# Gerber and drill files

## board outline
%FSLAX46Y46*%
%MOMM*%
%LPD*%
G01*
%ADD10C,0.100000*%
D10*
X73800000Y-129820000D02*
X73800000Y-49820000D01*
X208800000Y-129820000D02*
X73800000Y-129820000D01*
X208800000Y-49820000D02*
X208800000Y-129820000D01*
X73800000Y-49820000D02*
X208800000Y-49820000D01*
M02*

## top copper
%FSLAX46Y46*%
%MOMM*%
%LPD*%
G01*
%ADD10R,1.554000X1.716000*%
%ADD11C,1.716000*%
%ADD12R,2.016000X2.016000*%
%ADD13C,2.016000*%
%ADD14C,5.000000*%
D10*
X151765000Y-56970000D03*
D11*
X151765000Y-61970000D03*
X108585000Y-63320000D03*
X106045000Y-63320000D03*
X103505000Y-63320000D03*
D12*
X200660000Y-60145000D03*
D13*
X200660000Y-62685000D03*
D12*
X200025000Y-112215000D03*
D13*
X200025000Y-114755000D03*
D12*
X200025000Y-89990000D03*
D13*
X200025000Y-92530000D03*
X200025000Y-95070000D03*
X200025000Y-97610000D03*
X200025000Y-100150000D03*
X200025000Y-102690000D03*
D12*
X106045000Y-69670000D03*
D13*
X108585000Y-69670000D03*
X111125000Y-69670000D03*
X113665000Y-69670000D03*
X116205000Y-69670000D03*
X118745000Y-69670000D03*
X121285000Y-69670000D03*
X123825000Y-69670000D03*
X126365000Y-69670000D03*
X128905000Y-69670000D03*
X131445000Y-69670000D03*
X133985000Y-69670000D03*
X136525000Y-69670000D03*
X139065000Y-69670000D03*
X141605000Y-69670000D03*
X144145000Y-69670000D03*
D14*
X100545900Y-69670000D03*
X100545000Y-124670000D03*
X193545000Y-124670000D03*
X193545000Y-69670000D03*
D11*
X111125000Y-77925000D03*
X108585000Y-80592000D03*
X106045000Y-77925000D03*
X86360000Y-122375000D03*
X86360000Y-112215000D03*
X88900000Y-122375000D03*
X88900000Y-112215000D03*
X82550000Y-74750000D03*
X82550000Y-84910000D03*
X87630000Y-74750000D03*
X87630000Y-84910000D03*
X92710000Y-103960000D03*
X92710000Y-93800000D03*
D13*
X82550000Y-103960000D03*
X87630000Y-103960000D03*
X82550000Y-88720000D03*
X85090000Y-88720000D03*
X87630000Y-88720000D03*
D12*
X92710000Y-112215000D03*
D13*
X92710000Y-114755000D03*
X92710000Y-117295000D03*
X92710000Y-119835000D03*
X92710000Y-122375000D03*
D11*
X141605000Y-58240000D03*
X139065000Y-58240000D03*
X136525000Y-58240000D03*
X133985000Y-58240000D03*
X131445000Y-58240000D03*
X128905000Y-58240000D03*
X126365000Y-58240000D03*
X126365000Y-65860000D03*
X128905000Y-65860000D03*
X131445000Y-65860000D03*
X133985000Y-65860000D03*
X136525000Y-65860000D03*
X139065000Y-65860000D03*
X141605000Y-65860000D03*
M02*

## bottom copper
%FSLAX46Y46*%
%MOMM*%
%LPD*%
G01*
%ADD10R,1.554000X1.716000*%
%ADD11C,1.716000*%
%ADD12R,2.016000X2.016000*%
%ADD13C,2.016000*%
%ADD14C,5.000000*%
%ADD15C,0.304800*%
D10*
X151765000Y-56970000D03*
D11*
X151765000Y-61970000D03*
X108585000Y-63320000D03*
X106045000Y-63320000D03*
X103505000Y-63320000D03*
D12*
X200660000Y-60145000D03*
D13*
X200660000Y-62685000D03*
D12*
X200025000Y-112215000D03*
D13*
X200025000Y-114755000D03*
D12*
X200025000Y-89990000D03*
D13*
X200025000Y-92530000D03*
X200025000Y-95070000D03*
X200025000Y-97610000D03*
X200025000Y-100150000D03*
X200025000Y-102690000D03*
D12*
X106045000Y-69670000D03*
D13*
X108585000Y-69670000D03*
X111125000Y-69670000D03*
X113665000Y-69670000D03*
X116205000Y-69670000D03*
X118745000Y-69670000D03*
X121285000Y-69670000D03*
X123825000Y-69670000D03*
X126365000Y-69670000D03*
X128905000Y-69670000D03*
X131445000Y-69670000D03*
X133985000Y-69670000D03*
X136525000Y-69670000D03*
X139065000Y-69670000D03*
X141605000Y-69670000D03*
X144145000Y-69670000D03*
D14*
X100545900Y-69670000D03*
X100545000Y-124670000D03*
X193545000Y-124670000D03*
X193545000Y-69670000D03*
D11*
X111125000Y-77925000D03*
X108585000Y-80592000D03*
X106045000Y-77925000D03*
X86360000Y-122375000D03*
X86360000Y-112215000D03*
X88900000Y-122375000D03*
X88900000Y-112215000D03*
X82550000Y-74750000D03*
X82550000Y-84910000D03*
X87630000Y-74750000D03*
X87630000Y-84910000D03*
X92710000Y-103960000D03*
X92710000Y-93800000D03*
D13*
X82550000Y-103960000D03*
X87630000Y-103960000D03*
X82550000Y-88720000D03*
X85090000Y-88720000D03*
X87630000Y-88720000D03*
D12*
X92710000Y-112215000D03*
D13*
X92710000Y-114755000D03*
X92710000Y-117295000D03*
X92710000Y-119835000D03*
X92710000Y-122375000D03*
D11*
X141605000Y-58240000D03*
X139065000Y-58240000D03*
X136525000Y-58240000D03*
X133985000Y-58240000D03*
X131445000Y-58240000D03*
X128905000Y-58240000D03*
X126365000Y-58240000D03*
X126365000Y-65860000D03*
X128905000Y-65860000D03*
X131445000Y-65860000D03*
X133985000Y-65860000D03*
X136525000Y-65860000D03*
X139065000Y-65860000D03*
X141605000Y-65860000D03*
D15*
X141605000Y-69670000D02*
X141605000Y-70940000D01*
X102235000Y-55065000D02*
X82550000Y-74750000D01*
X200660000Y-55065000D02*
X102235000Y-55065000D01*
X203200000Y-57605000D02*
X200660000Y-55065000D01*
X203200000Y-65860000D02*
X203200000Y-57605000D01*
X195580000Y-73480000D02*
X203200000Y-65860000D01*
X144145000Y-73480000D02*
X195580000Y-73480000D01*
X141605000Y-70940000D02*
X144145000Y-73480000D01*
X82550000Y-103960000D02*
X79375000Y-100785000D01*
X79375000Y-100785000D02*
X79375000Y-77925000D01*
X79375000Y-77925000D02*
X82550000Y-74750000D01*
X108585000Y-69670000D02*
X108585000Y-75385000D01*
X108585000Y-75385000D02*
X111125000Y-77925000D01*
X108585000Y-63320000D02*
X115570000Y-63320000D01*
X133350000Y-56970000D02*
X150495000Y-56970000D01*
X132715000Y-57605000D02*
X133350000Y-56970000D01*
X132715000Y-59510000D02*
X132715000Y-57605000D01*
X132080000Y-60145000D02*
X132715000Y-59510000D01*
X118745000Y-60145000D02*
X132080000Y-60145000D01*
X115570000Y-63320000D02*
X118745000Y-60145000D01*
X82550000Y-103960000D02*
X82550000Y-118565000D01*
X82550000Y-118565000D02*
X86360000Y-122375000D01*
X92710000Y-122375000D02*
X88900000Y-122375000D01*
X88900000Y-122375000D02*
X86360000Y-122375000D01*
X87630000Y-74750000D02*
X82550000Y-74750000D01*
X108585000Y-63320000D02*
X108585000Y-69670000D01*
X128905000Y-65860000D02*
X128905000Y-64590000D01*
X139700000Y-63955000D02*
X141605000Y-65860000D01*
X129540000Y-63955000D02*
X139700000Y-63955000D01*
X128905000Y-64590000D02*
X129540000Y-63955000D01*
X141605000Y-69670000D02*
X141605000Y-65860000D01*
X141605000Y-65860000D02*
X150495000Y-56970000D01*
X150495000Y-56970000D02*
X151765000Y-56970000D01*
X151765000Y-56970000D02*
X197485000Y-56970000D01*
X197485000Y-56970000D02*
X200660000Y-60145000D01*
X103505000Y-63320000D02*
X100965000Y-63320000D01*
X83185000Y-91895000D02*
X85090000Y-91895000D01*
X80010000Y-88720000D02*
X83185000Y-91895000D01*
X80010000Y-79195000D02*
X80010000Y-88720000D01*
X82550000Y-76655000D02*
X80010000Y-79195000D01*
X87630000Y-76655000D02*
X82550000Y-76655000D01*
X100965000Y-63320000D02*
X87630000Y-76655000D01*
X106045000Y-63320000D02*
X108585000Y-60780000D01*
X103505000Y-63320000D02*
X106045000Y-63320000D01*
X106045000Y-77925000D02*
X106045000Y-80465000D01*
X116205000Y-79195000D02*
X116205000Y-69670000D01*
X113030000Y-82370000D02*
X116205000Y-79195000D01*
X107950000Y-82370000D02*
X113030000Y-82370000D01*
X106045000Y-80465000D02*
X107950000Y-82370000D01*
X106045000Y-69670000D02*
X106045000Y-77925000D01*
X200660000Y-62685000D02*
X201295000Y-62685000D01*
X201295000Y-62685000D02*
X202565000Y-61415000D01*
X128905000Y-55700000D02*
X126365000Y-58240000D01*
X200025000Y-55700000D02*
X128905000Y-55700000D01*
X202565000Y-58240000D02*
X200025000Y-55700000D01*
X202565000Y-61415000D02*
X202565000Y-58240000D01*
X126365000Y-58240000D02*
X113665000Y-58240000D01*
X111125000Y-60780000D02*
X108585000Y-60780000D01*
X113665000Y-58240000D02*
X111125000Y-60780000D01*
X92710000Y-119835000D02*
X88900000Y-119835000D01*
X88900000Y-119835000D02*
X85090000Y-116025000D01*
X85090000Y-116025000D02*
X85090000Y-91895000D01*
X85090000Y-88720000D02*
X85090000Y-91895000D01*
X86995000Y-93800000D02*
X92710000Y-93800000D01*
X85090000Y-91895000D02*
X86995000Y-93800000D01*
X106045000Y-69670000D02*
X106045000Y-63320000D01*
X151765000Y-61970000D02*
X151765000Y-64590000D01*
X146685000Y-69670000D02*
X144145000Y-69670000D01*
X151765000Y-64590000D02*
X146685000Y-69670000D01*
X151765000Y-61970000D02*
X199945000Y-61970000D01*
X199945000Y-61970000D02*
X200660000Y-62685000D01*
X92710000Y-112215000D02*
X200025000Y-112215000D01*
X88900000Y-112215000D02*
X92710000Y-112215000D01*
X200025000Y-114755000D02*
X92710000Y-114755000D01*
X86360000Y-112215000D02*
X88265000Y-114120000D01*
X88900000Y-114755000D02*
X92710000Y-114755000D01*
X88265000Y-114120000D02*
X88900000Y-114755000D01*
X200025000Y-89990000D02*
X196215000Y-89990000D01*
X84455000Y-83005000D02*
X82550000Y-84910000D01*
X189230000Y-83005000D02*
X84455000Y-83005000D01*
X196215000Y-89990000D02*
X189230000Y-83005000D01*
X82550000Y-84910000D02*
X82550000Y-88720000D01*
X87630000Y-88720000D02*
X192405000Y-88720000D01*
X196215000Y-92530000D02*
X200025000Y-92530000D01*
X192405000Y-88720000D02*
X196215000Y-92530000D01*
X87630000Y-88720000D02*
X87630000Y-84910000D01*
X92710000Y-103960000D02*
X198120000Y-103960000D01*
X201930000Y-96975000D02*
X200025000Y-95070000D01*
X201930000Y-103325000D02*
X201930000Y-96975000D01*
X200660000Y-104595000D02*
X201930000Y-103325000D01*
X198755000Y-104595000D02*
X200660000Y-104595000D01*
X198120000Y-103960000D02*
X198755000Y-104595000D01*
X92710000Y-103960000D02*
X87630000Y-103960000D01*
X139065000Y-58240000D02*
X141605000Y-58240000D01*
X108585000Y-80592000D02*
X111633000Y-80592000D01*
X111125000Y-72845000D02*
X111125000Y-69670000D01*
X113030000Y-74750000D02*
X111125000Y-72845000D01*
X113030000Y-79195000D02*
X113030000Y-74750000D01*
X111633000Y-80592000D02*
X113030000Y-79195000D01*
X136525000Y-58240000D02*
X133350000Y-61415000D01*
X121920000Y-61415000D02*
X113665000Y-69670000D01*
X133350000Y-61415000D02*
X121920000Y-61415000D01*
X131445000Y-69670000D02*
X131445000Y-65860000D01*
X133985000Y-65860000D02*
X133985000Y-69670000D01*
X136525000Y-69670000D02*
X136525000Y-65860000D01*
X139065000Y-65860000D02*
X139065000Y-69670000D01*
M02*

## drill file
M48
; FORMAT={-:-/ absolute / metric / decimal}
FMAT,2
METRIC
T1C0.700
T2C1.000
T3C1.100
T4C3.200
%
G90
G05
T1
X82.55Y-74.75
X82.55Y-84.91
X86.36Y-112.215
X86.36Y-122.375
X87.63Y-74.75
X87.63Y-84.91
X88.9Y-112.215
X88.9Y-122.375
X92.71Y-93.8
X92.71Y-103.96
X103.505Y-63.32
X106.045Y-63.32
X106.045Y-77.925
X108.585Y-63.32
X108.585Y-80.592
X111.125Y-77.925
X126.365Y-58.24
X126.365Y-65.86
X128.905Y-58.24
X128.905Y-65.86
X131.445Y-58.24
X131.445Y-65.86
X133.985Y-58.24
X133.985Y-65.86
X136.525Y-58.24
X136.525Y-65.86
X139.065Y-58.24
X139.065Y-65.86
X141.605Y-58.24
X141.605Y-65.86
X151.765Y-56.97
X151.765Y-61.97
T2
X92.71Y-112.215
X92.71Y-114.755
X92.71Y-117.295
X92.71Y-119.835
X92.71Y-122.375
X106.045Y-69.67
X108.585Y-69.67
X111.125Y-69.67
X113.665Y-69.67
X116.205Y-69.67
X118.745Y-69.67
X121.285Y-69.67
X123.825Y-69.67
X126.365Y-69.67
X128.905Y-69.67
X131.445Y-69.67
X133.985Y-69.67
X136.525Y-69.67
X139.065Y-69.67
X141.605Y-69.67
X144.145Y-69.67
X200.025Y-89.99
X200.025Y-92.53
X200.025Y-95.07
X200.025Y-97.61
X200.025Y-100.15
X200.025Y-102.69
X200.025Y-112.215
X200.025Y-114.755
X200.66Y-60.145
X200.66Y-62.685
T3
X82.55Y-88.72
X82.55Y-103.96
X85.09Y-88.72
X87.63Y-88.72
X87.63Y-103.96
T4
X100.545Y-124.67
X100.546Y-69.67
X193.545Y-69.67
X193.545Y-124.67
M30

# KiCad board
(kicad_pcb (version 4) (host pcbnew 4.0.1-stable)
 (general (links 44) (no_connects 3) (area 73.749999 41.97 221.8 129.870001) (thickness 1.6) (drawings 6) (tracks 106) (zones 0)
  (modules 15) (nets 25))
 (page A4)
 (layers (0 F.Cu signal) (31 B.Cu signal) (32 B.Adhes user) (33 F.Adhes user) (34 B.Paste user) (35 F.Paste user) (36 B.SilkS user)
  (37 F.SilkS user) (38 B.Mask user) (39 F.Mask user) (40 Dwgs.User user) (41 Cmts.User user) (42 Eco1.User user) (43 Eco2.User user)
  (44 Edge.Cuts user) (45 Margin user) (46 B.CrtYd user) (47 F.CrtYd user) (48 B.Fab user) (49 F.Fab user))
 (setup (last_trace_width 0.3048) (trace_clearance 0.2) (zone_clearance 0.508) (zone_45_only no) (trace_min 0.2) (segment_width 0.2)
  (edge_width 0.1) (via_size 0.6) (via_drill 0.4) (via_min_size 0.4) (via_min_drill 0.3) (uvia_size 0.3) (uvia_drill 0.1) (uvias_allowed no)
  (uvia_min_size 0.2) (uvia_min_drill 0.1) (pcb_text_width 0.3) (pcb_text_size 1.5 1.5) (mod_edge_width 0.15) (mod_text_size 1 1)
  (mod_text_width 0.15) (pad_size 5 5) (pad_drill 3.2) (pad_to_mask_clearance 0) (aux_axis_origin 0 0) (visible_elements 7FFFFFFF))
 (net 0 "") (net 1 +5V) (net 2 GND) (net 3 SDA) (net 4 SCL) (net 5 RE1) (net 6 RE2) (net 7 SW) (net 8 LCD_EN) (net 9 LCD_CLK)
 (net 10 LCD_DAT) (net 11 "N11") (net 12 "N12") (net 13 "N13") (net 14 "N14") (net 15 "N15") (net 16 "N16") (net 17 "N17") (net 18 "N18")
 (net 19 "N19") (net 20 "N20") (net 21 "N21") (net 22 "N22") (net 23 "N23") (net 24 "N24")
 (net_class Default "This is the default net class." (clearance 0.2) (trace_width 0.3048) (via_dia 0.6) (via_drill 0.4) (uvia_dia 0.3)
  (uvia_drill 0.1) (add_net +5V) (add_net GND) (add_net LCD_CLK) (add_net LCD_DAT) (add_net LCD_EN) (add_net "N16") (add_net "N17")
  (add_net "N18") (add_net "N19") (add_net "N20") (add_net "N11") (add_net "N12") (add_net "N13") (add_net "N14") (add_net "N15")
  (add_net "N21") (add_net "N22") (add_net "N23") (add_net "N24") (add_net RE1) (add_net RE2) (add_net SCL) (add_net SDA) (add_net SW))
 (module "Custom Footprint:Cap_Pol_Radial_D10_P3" (layer F.Cu) (at 151.765 56.97 270)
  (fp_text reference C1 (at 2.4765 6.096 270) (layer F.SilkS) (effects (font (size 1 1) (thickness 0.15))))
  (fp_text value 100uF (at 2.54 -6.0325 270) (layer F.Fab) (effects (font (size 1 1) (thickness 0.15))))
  (pad 1 thru_hole rect (at 0 0 270) (size 1.716 1.554) (drill 0.7) (layers *.Cu *.Mask F.SilkS) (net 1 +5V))
  (pad 2 thru_hole circle (at 5 0 270) (size 1.716 1.716) (drill 0.7) (layers *.Cu *.Mask F.SilkS) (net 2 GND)))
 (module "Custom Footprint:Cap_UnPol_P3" (layer F.Cu) (at 108.585 63.32 270)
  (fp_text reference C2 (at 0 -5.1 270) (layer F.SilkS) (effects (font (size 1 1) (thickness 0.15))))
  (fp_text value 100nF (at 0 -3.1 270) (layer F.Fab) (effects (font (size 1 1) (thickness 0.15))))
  (pad 1 thru_hole circle (at 0 0 270) (size 1.716 1.716) (drill 0.7) (layers *.Cu *.Mask F.SilkS) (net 1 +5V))
  (pad 2 thru_hole circle (at 0 2.54 270) (size 1.716 1.716) (drill 0.7) (layers *.Cu *.Mask F.SilkS) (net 2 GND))
  (pad 2 thru_hole circle (at 0 5.08 270) (size 1.716 1.716) (drill 0.7) (layers *.Cu *.Mask F.SilkS) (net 2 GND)))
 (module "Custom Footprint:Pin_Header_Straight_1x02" (layer F.Cu) (at 200.66 60.145)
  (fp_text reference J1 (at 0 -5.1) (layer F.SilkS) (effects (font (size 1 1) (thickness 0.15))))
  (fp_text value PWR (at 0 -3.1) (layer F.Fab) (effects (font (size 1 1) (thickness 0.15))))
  (pad 1 thru_hole rect (at 0 0) (size 2.016 2.016) (drill 1) (layers *.Cu *.Mask F.SilkS) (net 1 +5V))
  (pad 2 thru_hole circle (at 0 2.54) (size 2.016 2.016) (drill 1) (layers *.Cu *.Mask F.SilkS) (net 2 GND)))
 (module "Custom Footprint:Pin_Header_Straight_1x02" (layer F.Cu) (at 200.025 112.215)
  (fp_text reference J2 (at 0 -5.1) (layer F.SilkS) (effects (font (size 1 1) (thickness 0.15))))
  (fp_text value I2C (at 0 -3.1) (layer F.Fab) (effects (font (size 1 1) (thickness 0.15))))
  (pad 1 thru_hole rect (at 0 0) (size 2.016 2.016) (drill 1) (layers *.Cu *.Mask F.SilkS) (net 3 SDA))
  (pad 2 thru_hole circle (at 0 2.54) (size 2.016 2.016) (drill 1) (layers *.Cu *.Mask F.SilkS) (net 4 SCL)))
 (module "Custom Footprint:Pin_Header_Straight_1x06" (layer F.Cu) (at 200.025 89.99)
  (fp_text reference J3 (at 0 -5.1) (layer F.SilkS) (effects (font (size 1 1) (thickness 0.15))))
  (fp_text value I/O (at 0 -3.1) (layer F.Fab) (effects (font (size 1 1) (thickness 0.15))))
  (pad 1 thru_hole rect (at 0 0) (size 2.016 2.016) (drill 1) (layers *.Cu *.Mask F.SilkS) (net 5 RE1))
  (pad 2 thru_hole circle (at 0 2.54) (size 2.016 2.016) (drill 1) (layers *.Cu *.Mask F.SilkS) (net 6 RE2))
  (pad 3 thru_hole circle (at 0 5.08) (size 2.016 2.016) (drill 1) (layers *.Cu *.Mask F.SilkS) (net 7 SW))
  (pad 4 thru_hole circle (at 0 7.62) (size 2.016 2.016) (drill 1) (layers *.Cu *.Mask F.SilkS) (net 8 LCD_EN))
  (pad 5 thru_hole circle (at 0 10.16) (size 2.016 2.016) (drill 1) (layers *.Cu *.Mask F.SilkS) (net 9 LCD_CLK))
  (pad 6 thru_hole circle (at 0 12.7) (size 2.016 2.016) (drill 1) (layers *.Cu *.Mask F.SilkS) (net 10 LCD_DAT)))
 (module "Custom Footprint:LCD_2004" (layer F.Cu) (at 106.045 69.67)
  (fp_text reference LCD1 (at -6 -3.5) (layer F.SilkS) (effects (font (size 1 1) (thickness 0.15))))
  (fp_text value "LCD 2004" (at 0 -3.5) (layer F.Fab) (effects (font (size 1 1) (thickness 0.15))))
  (pad 1 thru_hole rect (at 0 0) (size 2.016 2.016) (drill 1) (layers *.Cu *.Mask F.SilkS) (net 2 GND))
  (pad 2 thru_hole circle (at 2.54 0) (size 2.016 2.016) (drill 1) (layers *.Cu *.Mask F.SilkS) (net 1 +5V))
  (pad 3 thru_hole circle (at 5.08 0) (size 2.016 2.016) (drill 1) (layers *.Cu *.Mask F.SilkS) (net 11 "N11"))
  (pad 4 thru_hole circle (at 7.62 0) (size 2.016 2.016) (drill 1) (layers *.Cu *.Mask F.SilkS) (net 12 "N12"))
  (pad 5 thru_hole circle (at 10.16 0) (size 2.016 2.016) (drill 1) (layers *.Cu *.Mask F.SilkS) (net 2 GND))
  (pad 6 thru_hole circle (at 12.7 0) (size 2.016 2.016) (drill 1) (layers *.Cu *.Mask F.SilkS) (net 8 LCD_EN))
  (pad 7 thru_hole circle (at 15.24 0) (size 2.016 2.016) (drill 1) (layers *.Cu *.Mask F.SilkS) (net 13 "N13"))
  (pad 8 thru_hole circle (at 17.78 0) (size 2.016 2.016) (drill 1) (layers *.Cu *.Mask F.SilkS) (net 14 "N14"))
  (pad 9 thru_hole circle (at 20.32 0) (size 2.016 2.016) (drill 1) (layers *.Cu *.Mask F.SilkS) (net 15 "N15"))
  (pad 10 thru_hole circle (at 22.86 0) (size 2.016 2.016) (drill 1) (layers *.Cu *.Mask F.SilkS) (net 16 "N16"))
  (pad 11 thru_hole circle (at 25.4 0) (size 2.016 2.016) (drill 1) (layers *.Cu *.Mask F.SilkS) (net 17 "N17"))
  (pad 12 thru_hole circle (at 27.94 0) (size 2.016 2.016) (drill 1) (layers *.Cu *.Mask F.SilkS) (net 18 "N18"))
  (pad 13 thru_hole circle (at 30.48 0) (size 2.016 2.016) (drill 1) (layers *.Cu *.Mask F.SilkS) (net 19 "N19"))
  (pad 14 thru_hole circle (at 33.02 0) (size 2.016 2.016) (drill 1) (layers *.Cu *.Mask F.SilkS) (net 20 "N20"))
  (pad 15 thru_hole circle (at 35.56 0) (size 2.016 2.016) (drill 1) (layers *.Cu *.Mask F.SilkS) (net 1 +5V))
  (pad 16 thru_hole circle (at 38.1 0) (size 2.016 2.016) (drill 1) (layers *.Cu *.Mask F.SilkS) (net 2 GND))
  (pad 0 thru_hole circle (at -5.4991 0) (size 5 5) (drill 3.2) (layers *.Cu *.Mask F.SilkS))
  (pad 0 thru_hole circle (at -5.5 55) (size 5 5) (drill 3.2) (layers *.Cu *.Mask F.SilkS))
  (pad 0 thru_hole circle (at 87.5 55) (size 5 5) (drill 3.2) (layers *.Cu *.Mask F.SilkS))
  (pad 0 thru_hole circle (at 87.5 0) (size 5 5) (drill 3.2) (layers *.Cu *.Mask F.SilkS)))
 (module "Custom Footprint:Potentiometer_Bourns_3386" (layer F.Cu) (at 111.125 77.925)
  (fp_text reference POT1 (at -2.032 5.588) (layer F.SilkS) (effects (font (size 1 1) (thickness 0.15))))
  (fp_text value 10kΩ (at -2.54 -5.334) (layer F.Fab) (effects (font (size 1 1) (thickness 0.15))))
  (pad 1 thru_hole circle (at 0 0) (size 1.716 1.716) (drill 0.7) (layers *.Cu *.Mask F.SilkS) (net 1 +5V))
  (pad 2 thru_hole circle (at -2.54 2.667) (size 1.716 1.716) (drill 0.7) (layers *.Cu *.Mask F.SilkS) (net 11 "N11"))
  (pad 3 thru_hole circle (at -5.08 0) (size 1.716 1.716) (drill 0.7) (layers *.Cu *.Mask F.SilkS) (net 2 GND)))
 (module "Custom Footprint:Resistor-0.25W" (layer F.Cu) (at 86.36 122.375 90)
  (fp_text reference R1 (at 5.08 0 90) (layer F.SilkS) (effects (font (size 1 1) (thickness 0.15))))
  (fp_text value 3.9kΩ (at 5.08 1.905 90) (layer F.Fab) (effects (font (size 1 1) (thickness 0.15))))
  (pad 1 thru_hole circle (at 0 0 90) (size 1.716 1.716) (drill 0.7) (layers *.Cu *.Mask F.SilkS) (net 1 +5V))
  (pad 2 thru_hole circle (at 10.16 0 90) (size 1.716 1.716) (drill 0.7) (layers *.Cu *.Mask F.SilkS) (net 4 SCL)))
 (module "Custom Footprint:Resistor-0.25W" (layer F.Cu) (at 88.9 122.375 90)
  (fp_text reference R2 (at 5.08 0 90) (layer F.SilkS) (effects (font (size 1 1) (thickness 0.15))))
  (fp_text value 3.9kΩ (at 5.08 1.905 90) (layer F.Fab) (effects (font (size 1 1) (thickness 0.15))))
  (pad 1 thru_hole circle (at 0 0 90) (size 1.716 1.716) (drill 0.7) (layers *.Cu *.Mask F.SilkS) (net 1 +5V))
  (pad 2 thru_hole circle (at 10.16 0 90) (size 1.716 1.716) (drill 0.7) (layers *.Cu *.Mask F.SilkS) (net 3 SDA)))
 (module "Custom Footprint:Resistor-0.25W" (layer F.Cu) (at 82.55 74.75 270)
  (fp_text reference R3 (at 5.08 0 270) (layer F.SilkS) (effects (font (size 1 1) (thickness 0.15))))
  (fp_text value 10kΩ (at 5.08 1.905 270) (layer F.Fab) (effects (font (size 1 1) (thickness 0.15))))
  (pad 1 thru_hole circle (at 0 0 270) (size 1.716 1.716) (drill 0.7) (layers *.Cu *.Mask F.SilkS) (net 1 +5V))
  (pad 2 thru_hole circle (at 10.16 0 270) (size 1.716 1.716) (drill 0.7) (layers *.Cu *.Mask F.SilkS) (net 5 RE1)))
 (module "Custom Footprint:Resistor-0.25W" (layer F.Cu) (at 87.63 74.75 270)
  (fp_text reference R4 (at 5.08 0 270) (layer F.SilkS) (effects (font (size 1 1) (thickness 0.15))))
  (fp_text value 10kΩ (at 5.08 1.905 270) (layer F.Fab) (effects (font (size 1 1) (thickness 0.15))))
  (pad 1 thru_hole circle (at 0 0 270) (size 1.716 1.716) (drill 0.7) (layers *.Cu *.Mask F.SilkS) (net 1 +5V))
  (pad 2 thru_hole circle (at 10.16 0 270) (size 1.716 1.716) (drill 0.7) (layers *.Cu *.Mask F.SilkS) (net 6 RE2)))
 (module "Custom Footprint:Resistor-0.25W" (layer F.Cu) (at 92.71 103.96 90)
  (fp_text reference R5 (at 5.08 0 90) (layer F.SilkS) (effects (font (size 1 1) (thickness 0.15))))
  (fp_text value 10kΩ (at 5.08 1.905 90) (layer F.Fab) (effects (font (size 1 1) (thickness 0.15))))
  (pad 1 thru_hole circle (at 0 0 90) (size 1.716 1.716) (drill 0.7) (layers *.Cu *.Mask F.SilkS) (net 7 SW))
  (pad 2 thru_hole circle (at 10.16 0 90) (size 1.716 1.716) (drill 0.7) (layers *.Cu *.Mask F.SilkS) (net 2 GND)))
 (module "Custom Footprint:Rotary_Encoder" (layer F.Cu) (at 85.09 98.88 180)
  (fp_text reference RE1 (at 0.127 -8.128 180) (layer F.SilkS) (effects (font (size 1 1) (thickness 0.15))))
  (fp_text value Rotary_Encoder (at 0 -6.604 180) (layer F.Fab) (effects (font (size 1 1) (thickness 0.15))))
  (pad 1 thru_hole circle (at 2.54 -5.08 180) (size 2.016 2.016) (drill 1.1) (layers *.Cu *.Mask F.SilkS) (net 1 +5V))
  (pad 2 thru_hole circle (at -2.54 -5.08 180) (size 2.016 2.016) (drill 1.1) (layers *.Cu *.Mask F.SilkS) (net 7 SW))
  (pad 3 thru_hole circle (at 2.54 10.16 180) (size 2.016 2.016) (drill 1.1) (layers *.Cu *.Mask F.SilkS) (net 5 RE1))
  (pad 4 thru_hole circle (at 0 10.16 180) (size 2.016 2.016) (drill 1.1) (layers *.Cu *.Mask F.SilkS) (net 2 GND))
  (pad 5 thru_hole circle (at -2.54 10.16 180) (size 2.016 2.016) (drill 1.1) (layers *.Cu *.Mask F.SilkS) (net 6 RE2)))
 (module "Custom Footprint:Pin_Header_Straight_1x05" (layer F.Cu) (at 92.71 112.215)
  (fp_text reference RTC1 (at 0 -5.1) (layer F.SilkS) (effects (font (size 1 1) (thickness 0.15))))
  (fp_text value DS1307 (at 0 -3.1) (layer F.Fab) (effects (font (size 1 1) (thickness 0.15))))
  (pad 1 thru_hole rect (at 0 0) (size 2.016 2.016) (drill 1) (layers *.Cu *.Mask F.SilkS) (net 3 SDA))
  (pad 2 thru_hole circle (at 0 2.54) (size 2.016 2.016) (drill 1) (layers *.Cu *.Mask F.SilkS) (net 4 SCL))
  (pad 3 thru_hole circle (at 0 5.08) (size 2.016 2.016) (drill 1) (layers *.Cu *.Mask F.SilkS) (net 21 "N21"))
  (pad 4 thru_hole circle (at 0 7.62) (size 2.016 2.016) (drill 1) (layers *.Cu *.Mask F.SilkS) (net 2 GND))
  (pad 5 thru_hole circle (at 0 10.16) (size 2.016 2.016) (drill 1) (layers *.Cu *.Mask F.SilkS) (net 1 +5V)))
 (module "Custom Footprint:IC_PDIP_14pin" (layer F.Cu) (at 141.605 58.24 270)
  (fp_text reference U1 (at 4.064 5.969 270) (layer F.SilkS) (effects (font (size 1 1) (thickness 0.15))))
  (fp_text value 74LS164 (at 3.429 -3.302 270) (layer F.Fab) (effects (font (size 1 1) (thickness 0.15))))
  (pad 1 thru_hole circle (at 0 0 270) (size 1.716 1.716) (drill 0.7) (layers *.Cu *.Mask F.SilkS) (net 10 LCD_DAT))
  (pad 2 thru_hole circle (at 0 2.54 270) (size 1.716 1.716) (drill 0.7) (layers *.Cu *.Mask F.SilkS) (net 10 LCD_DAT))
  (pad 3 thru_hole circle (at 0 5.08 270) (size 1.716 1.716) (drill 0.7) (layers *.Cu *.Mask F.SilkS) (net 12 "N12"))
  (pad 4 thru_hole circle (at 0 7.62 270) (size 1.716 1.716) (drill 0.7) (layers *.Cu *.Mask F.SilkS) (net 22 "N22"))
  (pad 5 thru_hole circle (at 0 10.16 270) (size 1.716 1.716) (drill 0.7) (layers *.Cu *.Mask F.SilkS) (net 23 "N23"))
  (pad 6 thru_hole circle (at 0 12.7 270) (size 1.716 1.716) (drill 0.7) (layers *.Cu *.Mask F.SilkS) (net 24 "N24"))
  (pad 7 thru_hole circle (at 0 15.24 270) (size 1.716 1.716) (drill 0.7) (layers *.Cu *.Mask F.SilkS) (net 2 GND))
  (pad 8 thru_hole circle (at 7.62 15.24 270) (size 1.716 1.716) (drill 0.7) (layers *.Cu *.Mask F.SilkS) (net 9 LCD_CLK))
  (pad 9 thru_hole circle (at 7.62 12.7 270) (size 1.716 1.716) (drill 0.7) (layers *.Cu *.Mask F.SilkS) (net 1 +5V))
  (pad 10 thru_hole circle (at 7.62 10.16 270) (size 1.716 1.716) (drill 0.7) (layers *.Cu *.Mask F.SilkS) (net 17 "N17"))
  (pad 11 thru_hole circle (at 7.62 7.62 270) (size 1.716 1.716) (drill 0.7) (layers *.Cu *.Mask F.SilkS) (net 18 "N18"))
  (pad 12 thru_hole circle (at 7.62 5.08 270) (size 1.716 1.716) (drill 0.7) (layers *.Cu *.Mask F.SilkS) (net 19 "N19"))
  (pad 13 thru_hole circle (at 7.62 2.54 270) (size 1.716 1.716) (drill 0.7) (layers *.Cu *.Mask F.SilkS) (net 20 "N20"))
  (pad 14 thru_hole circle (at 7.62 0 270) (size 1.716 1.716) (drill 0.7) (layers *.Cu *.Mask F.SilkS) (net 1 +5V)))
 (gr_line (start 73.8 129.82) (end 73.8 49.82) (angle 90) (layer Edge.Cuts) (width 0.1))
 (gr_line (start 208.8 129.82) (end 73.8 129.82) (angle 90) (layer Edge.Cuts) (width 0.1))
 (gr_line (start 208.8 49.82) (end 208.8 129.82) (angle 90) (layer Edge.Cuts) (width 0.1))
 (gr_line (start 73.8 49.82) (end 208.8 49.82) (angle 90) (layer Edge.Cuts) (width 0.1))
 (segment (start 141.605 69.67) (end 141.605 70.94) (width 0.3048) (layer B.Cu) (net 1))
 (segment (start 102.235 55.065) (end 82.55 74.75) (width 0.3048) (layer B.Cu) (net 1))
 (segment (start 200.66 55.065) (end 102.235 55.065) (width 0.3048) (layer B.Cu) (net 1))
 (segment (start 203.2 57.605) (end 200.66 55.065) (width 0.3048) (layer B.Cu) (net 1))
 (segment (start 203.2 65.86) (end 203.2 57.605) (width 0.3048) (layer B.Cu) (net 1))
 (segment (start 195.58 73.48) (end 203.2 65.86) (width 0.3048) (layer B.Cu) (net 1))
 (segment (start 144.145 73.48) (end 195.58 73.48) (width 0.3048) (layer B.Cu) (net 1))
 (segment (start 141.605 70.94) (end 144.145 73.48) (width 0.3048) (layer B.Cu) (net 1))
 (segment (start 82.55 103.96) (end 79.375 100.785) (width 0.3048) (layer B.Cu) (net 1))
 (segment (start 79.375 100.785) (end 79.375 77.925) (width 0.3048) (layer B.Cu) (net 1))
 (segment (start 79.375 77.925) (end 82.55 74.75) (width 0.3048) (layer B.Cu) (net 1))
 (segment (start 108.585 69.67) (end 108.585 75.385) (width 0.3048) (layer B.Cu) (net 1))
 (segment (start 108.585 75.385) (end 111.125 77.925) (width 0.3048) (layer B.Cu) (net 1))
 (segment (start 108.585 63.32) (end 115.57 63.32) (width 0.3048) (layer B.Cu) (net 1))
 (segment (start 133.35 56.97) (end 150.495 56.97) (width 0.3048) (layer B.Cu) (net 1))
 (segment (start 132.715 57.605) (end 133.35 56.97) (width 0.3048) (layer B.Cu) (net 1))
 (segment (start 132.715 59.51) (end 132.715 57.605) (width 0.3048) (layer B.Cu) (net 1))
 (segment (start 132.08 60.145) (end 132.715 59.51) (width 0.3048) (layer B.Cu) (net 1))
 (segment (start 118.745 60.145) (end 132.08 60.145) (width 0.3048) (layer B.Cu) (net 1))
 (segment (start 115.57 63.32) (end 118.745 60.145) (width 0.3048) (layer B.Cu) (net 1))
 (segment (start 82.55 103.96) (end 82.55 118.565) (width 0.3048) (layer B.Cu) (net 1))
 (segment (start 82.55 118.565) (end 86.36 122.375) (width 0.3048) (layer B.Cu) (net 1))
 (segment (start 92.71 122.375) (end 88.9 122.375) (width 0.3048) (layer B.Cu) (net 1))
 (segment (start 88.9 122.375) (end 86.36 122.375) (width 0.3048) (layer B.Cu) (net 1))
 (segment (start 87.63 74.75) (end 82.55 74.75) (width 0.3048) (layer B.Cu) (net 1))
 (segment (start 108.585 63.32) (end 108.585 69.67) (width 0.3048) (layer B.Cu) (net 1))
 (segment (start 128.905 65.86) (end 128.905 64.59) (width 0.3048) (layer B.Cu) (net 1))
 (segment (start 139.7 63.955) (end 141.605 65.86) (width 0.3048) (layer B.Cu) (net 1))
 (segment (start 129.54 63.955) (end 139.7 63.955) (width 0.3048) (layer B.Cu) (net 1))
 (segment (start 128.905 64.59) (end 129.54 63.955) (width 0.3048) (layer B.Cu) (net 1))
 (segment (start 141.605 69.67) (end 141.605 65.86) (width 0.3048) (layer B.Cu) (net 1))
 (segment (start 141.605 65.86) (end 150.495 56.97) (width 0.3048) (layer B.Cu) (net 1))
 (segment (start 150.495 56.97) (end 151.765 56.97) (width 0.3048) (layer B.Cu) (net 1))
 (segment (start 151.765 56.97) (end 197.485 56.97) (width 0.3048) (layer B.Cu) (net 1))
 (segment (start 197.485 56.97) (end 200.66 60.145) (width 0.3048) (layer B.Cu) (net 1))
 (segment (start 103.505 63.32) (end 100.965 63.32) (width 0.3048) (layer B.Cu) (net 2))
 (segment (start 83.185 91.895) (end 85.09 91.895) (width 0.3048) (layer B.Cu) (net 2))
 (segment (start 80.01 88.72) (end 83.185 91.895) (width 0.3048) (layer B.Cu) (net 2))
 (segment (start 80.01 79.195) (end 80.01 88.72) (width 0.3048) (layer B.Cu) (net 2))
 (segment (start 82.55 76.655) (end 80.01 79.195) (width 0.3048) (layer B.Cu) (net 2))
 (segment (start 87.63 76.655) (end 82.55 76.655) (width 0.3048) (layer B.Cu) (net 2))
 (segment (start 100.965 63.32) (end 87.63 76.655) (width 0.3048) (layer B.Cu) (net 2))
 (segment (start 106.045 63.32) (end 108.585 60.78) (width 0.3048) (layer B.Cu) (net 2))
 (segment (start 103.505 63.32) (end 106.045 63.32) (width 0.3048) (layer B.Cu) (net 2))
 (segment (start 106.045 77.925) (end 106.045 80.465) (width 0.3048) (layer B.Cu) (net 2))
 (segment (start 116.205 79.195) (end 116.205 69.67) (width 0.3048) (layer B.Cu) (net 2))
 (segment (start 113.03 82.37) (end 116.205 79.195) (width 0.3048) (layer B.Cu) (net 2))
 (segment (start 107.95 82.37) (end 113.03 82.37) (width 0.3048) (layer B.Cu) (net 2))
 (segment (start 106.045 80.465) (end 107.95 82.37) (width 0.3048) (layer B.Cu) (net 2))
 (segment (start 106.045 69.67) (end 106.045 77.925) (width 0.3048) (layer B.Cu) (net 2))
 (segment (start 200.66 62.685) (end 201.295 62.685) (width 0.3048) (layer B.Cu) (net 2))
 (segment (start 201.295 62.685) (end 202.565 61.415) (width 0.3048) (layer B.Cu) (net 2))
 (segment (start 128.905 55.7) (end 126.365 58.24) (width 0.3048) (layer B.Cu) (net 2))
 (segment (start 200.025 55.7) (end 128.905 55.7) (width 0.3048) (layer B.Cu) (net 2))
 (segment (start 202.565 58.24) (end 200.025 55.7) (width 0.3048) (layer B.Cu) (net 2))
 (segment (start 202.565 61.415) (end 202.565 58.24) (width 0.3048) (layer B.Cu) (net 2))
 (segment (start 126.365 58.24) (end 113.665 58.24) (width 0.3048) (layer B.Cu) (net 2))
 (segment (start 111.125 60.78) (end 108.585 60.78) (width 0.3048) (layer B.Cu) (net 2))
 (segment (start 113.665 58.24) (end 111.125 60.78) (width 0.3048) (layer B.Cu) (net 2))
 (segment (start 92.71 119.835) (end 88.9 119.835) (width 0.3048) (layer B.Cu) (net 2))
 (segment (start 88.9 119.835) (end 85.09 116.025) (width 0.3048) (layer B.Cu) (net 2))
 (segment (start 85.09 116.025) (end 85.09 91.895) (width 0.3048) (layer B.Cu) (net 2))
 (segment (start 85.09 88.72) (end 85.09 91.895) (width 0.3048) (layer B.Cu) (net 2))
 (segment (start 86.995 93.8) (end 92.71 93.8) (width 0.3048) (layer B.Cu) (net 2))
 (segment (start 85.09 91.895) (end 86.995 93.8) (width 0.3048) (layer B.Cu) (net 2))
 (segment (start 106.045 69.67) (end 106.045 63.32) (width 0.3048) (layer B.Cu) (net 2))
 (segment (start 151.765 61.97) (end 151.765 64.59) (width 0.3048) (layer B.Cu) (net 2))
 (segment (start 146.685 69.67) (end 144.145 69.67) (width 0.3048) (layer B.Cu) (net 2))
 (segment (start 151.765 64.59) (end 146.685 69.67) (width 0.3048) (layer B.Cu) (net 2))
 (segment (start 151.765 61.97) (end 199.945 61.97) (width 0.3048) (layer B.Cu) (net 2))
 (segment (start 199.945 61.97) (end 200.66 62.685) (width 0.3048) (layer B.Cu) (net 2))
 (segment (start 92.71 112.215) (end 200.025 112.215) (width 0.3048) (layer B.Cu) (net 3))
 (segment (start 88.9 112.215) (end 92.71 112.215) (width 0.3048) (layer B.Cu) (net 3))
 (segment (start 200.025 114.755) (end 92.71 114.755) (width 0.3048) (layer B.Cu) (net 4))
 (segment (start 86.36 112.215) (end 88.265 114.12) (width 0.3048) (layer B.Cu) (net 4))
 (segment (start 88.9 114.755) (end 92.71 114.755) (width 0.3048) (layer B.Cu) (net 4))
 (segment (start 88.265 114.12) (end 88.9 114.755) (width 0.3048) (layer B.Cu) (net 4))
 (segment (start 200.025 89.99) (end 196.215 89.99) (width 0.3048) (layer B.Cu) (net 5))
 (segment (start 84.455 83.005) (end 82.55 84.91) (width 0.3048) (layer B.Cu) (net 5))
 (segment (start 189.23 83.005) (end 84.455 83.005) (width 0.3048) (layer B.Cu) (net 5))
 (segment (start 196.215 89.99) (end 189.23 83.005) (width 0.3048) (layer B.Cu) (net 5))
 (segment (start 82.55 84.91) (end 82.55 88.72) (width 0.3048) (layer B.Cu) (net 5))
 (segment (start 87.63 88.72) (end 192.405 88.72) (width 0.3048) (layer B.Cu) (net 6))
 (segment (start 196.215 92.53) (end 200.025 92.53) (width 0.3048) (layer B.Cu) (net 6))
 (segment (start 192.405 88.72) (end 196.215 92.53) (width 0.3048) (layer B.Cu) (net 6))
 (segment (start 87.63 88.72) (end 87.63 84.91) (width 0.3048) (layer B.Cu) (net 6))
 (segment (start 92.71 103.96) (end 198.12 103.96) (width 0.3048) (layer B.Cu) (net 7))
 (segment (start 201.93 96.975) (end 200.025 95.07) (width 0.3048) (layer B.Cu) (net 7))
 (segment (start 201.93 103.325) (end 201.93 96.975) (width 0.3048) (layer B.Cu) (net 7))
 (segment (start 200.66 104.595) (end 201.93 103.325) (width 0.3048) (layer B.Cu) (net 7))
 (segment (start 198.755 104.595) (end 200.66 104.595) (width 0.3048) (layer B.Cu) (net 7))
 (segment (start 198.12 103.96) (end 198.755 104.595) (width 0.3048) (layer B.Cu) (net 7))
 (segment (start 92.71 103.96) (end 87.63 103.96) (width 0.3048) (layer B.Cu) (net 7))
 (segment (start 139.065 58.24) (end 141.605 58.24) (width 0.3048) (layer B.Cu) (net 10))
 (segment (start 108.585 80.592) (end 111.633 80.592) (width 0.3048) (layer B.Cu) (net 11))
 (segment (start 111.125 72.845) (end 111.125 69.67) (width 0.3048) (layer B.Cu) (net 11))
 (segment (start 113.03 74.75) (end 111.125 72.845) (width 0.3048) (layer B.Cu) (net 11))
 (segment (start 113.03 79.195) (end 113.03 74.75) (width 0.3048) (layer B.Cu) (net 11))
 (segment (start 111.633 80.592) (end 113.03 79.195) (width 0.3048) (layer B.Cu) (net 11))
 (segment (start 136.525 58.24) (end 133.35 61.415) (width 0.3048) (layer B.Cu) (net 12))
 (segment (start 121.92 61.415) (end 113.665 69.67) (width 0.3048) (layer B.Cu) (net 12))
 (segment (start 133.35 61.415) (end 121.92 61.415) (width 0.3048) (layer B.Cu) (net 12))
 (segment (start 131.445 69.67) (end 131.445 65.86) (width 0.3048) (layer B.Cu) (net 17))
 (segment (start 133.985 65.86) (end 133.985 69.67) (width 0.3048) (layer B.Cu) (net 18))
 (segment (start 136.525 69.67) (end 136.525 65.86) (width 0.3048) (layer B.Cu) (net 19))
 (segment (start 139.065 65.86) (end 139.065 69.67) (width 0.3048) (layer B.Cu) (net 20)))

